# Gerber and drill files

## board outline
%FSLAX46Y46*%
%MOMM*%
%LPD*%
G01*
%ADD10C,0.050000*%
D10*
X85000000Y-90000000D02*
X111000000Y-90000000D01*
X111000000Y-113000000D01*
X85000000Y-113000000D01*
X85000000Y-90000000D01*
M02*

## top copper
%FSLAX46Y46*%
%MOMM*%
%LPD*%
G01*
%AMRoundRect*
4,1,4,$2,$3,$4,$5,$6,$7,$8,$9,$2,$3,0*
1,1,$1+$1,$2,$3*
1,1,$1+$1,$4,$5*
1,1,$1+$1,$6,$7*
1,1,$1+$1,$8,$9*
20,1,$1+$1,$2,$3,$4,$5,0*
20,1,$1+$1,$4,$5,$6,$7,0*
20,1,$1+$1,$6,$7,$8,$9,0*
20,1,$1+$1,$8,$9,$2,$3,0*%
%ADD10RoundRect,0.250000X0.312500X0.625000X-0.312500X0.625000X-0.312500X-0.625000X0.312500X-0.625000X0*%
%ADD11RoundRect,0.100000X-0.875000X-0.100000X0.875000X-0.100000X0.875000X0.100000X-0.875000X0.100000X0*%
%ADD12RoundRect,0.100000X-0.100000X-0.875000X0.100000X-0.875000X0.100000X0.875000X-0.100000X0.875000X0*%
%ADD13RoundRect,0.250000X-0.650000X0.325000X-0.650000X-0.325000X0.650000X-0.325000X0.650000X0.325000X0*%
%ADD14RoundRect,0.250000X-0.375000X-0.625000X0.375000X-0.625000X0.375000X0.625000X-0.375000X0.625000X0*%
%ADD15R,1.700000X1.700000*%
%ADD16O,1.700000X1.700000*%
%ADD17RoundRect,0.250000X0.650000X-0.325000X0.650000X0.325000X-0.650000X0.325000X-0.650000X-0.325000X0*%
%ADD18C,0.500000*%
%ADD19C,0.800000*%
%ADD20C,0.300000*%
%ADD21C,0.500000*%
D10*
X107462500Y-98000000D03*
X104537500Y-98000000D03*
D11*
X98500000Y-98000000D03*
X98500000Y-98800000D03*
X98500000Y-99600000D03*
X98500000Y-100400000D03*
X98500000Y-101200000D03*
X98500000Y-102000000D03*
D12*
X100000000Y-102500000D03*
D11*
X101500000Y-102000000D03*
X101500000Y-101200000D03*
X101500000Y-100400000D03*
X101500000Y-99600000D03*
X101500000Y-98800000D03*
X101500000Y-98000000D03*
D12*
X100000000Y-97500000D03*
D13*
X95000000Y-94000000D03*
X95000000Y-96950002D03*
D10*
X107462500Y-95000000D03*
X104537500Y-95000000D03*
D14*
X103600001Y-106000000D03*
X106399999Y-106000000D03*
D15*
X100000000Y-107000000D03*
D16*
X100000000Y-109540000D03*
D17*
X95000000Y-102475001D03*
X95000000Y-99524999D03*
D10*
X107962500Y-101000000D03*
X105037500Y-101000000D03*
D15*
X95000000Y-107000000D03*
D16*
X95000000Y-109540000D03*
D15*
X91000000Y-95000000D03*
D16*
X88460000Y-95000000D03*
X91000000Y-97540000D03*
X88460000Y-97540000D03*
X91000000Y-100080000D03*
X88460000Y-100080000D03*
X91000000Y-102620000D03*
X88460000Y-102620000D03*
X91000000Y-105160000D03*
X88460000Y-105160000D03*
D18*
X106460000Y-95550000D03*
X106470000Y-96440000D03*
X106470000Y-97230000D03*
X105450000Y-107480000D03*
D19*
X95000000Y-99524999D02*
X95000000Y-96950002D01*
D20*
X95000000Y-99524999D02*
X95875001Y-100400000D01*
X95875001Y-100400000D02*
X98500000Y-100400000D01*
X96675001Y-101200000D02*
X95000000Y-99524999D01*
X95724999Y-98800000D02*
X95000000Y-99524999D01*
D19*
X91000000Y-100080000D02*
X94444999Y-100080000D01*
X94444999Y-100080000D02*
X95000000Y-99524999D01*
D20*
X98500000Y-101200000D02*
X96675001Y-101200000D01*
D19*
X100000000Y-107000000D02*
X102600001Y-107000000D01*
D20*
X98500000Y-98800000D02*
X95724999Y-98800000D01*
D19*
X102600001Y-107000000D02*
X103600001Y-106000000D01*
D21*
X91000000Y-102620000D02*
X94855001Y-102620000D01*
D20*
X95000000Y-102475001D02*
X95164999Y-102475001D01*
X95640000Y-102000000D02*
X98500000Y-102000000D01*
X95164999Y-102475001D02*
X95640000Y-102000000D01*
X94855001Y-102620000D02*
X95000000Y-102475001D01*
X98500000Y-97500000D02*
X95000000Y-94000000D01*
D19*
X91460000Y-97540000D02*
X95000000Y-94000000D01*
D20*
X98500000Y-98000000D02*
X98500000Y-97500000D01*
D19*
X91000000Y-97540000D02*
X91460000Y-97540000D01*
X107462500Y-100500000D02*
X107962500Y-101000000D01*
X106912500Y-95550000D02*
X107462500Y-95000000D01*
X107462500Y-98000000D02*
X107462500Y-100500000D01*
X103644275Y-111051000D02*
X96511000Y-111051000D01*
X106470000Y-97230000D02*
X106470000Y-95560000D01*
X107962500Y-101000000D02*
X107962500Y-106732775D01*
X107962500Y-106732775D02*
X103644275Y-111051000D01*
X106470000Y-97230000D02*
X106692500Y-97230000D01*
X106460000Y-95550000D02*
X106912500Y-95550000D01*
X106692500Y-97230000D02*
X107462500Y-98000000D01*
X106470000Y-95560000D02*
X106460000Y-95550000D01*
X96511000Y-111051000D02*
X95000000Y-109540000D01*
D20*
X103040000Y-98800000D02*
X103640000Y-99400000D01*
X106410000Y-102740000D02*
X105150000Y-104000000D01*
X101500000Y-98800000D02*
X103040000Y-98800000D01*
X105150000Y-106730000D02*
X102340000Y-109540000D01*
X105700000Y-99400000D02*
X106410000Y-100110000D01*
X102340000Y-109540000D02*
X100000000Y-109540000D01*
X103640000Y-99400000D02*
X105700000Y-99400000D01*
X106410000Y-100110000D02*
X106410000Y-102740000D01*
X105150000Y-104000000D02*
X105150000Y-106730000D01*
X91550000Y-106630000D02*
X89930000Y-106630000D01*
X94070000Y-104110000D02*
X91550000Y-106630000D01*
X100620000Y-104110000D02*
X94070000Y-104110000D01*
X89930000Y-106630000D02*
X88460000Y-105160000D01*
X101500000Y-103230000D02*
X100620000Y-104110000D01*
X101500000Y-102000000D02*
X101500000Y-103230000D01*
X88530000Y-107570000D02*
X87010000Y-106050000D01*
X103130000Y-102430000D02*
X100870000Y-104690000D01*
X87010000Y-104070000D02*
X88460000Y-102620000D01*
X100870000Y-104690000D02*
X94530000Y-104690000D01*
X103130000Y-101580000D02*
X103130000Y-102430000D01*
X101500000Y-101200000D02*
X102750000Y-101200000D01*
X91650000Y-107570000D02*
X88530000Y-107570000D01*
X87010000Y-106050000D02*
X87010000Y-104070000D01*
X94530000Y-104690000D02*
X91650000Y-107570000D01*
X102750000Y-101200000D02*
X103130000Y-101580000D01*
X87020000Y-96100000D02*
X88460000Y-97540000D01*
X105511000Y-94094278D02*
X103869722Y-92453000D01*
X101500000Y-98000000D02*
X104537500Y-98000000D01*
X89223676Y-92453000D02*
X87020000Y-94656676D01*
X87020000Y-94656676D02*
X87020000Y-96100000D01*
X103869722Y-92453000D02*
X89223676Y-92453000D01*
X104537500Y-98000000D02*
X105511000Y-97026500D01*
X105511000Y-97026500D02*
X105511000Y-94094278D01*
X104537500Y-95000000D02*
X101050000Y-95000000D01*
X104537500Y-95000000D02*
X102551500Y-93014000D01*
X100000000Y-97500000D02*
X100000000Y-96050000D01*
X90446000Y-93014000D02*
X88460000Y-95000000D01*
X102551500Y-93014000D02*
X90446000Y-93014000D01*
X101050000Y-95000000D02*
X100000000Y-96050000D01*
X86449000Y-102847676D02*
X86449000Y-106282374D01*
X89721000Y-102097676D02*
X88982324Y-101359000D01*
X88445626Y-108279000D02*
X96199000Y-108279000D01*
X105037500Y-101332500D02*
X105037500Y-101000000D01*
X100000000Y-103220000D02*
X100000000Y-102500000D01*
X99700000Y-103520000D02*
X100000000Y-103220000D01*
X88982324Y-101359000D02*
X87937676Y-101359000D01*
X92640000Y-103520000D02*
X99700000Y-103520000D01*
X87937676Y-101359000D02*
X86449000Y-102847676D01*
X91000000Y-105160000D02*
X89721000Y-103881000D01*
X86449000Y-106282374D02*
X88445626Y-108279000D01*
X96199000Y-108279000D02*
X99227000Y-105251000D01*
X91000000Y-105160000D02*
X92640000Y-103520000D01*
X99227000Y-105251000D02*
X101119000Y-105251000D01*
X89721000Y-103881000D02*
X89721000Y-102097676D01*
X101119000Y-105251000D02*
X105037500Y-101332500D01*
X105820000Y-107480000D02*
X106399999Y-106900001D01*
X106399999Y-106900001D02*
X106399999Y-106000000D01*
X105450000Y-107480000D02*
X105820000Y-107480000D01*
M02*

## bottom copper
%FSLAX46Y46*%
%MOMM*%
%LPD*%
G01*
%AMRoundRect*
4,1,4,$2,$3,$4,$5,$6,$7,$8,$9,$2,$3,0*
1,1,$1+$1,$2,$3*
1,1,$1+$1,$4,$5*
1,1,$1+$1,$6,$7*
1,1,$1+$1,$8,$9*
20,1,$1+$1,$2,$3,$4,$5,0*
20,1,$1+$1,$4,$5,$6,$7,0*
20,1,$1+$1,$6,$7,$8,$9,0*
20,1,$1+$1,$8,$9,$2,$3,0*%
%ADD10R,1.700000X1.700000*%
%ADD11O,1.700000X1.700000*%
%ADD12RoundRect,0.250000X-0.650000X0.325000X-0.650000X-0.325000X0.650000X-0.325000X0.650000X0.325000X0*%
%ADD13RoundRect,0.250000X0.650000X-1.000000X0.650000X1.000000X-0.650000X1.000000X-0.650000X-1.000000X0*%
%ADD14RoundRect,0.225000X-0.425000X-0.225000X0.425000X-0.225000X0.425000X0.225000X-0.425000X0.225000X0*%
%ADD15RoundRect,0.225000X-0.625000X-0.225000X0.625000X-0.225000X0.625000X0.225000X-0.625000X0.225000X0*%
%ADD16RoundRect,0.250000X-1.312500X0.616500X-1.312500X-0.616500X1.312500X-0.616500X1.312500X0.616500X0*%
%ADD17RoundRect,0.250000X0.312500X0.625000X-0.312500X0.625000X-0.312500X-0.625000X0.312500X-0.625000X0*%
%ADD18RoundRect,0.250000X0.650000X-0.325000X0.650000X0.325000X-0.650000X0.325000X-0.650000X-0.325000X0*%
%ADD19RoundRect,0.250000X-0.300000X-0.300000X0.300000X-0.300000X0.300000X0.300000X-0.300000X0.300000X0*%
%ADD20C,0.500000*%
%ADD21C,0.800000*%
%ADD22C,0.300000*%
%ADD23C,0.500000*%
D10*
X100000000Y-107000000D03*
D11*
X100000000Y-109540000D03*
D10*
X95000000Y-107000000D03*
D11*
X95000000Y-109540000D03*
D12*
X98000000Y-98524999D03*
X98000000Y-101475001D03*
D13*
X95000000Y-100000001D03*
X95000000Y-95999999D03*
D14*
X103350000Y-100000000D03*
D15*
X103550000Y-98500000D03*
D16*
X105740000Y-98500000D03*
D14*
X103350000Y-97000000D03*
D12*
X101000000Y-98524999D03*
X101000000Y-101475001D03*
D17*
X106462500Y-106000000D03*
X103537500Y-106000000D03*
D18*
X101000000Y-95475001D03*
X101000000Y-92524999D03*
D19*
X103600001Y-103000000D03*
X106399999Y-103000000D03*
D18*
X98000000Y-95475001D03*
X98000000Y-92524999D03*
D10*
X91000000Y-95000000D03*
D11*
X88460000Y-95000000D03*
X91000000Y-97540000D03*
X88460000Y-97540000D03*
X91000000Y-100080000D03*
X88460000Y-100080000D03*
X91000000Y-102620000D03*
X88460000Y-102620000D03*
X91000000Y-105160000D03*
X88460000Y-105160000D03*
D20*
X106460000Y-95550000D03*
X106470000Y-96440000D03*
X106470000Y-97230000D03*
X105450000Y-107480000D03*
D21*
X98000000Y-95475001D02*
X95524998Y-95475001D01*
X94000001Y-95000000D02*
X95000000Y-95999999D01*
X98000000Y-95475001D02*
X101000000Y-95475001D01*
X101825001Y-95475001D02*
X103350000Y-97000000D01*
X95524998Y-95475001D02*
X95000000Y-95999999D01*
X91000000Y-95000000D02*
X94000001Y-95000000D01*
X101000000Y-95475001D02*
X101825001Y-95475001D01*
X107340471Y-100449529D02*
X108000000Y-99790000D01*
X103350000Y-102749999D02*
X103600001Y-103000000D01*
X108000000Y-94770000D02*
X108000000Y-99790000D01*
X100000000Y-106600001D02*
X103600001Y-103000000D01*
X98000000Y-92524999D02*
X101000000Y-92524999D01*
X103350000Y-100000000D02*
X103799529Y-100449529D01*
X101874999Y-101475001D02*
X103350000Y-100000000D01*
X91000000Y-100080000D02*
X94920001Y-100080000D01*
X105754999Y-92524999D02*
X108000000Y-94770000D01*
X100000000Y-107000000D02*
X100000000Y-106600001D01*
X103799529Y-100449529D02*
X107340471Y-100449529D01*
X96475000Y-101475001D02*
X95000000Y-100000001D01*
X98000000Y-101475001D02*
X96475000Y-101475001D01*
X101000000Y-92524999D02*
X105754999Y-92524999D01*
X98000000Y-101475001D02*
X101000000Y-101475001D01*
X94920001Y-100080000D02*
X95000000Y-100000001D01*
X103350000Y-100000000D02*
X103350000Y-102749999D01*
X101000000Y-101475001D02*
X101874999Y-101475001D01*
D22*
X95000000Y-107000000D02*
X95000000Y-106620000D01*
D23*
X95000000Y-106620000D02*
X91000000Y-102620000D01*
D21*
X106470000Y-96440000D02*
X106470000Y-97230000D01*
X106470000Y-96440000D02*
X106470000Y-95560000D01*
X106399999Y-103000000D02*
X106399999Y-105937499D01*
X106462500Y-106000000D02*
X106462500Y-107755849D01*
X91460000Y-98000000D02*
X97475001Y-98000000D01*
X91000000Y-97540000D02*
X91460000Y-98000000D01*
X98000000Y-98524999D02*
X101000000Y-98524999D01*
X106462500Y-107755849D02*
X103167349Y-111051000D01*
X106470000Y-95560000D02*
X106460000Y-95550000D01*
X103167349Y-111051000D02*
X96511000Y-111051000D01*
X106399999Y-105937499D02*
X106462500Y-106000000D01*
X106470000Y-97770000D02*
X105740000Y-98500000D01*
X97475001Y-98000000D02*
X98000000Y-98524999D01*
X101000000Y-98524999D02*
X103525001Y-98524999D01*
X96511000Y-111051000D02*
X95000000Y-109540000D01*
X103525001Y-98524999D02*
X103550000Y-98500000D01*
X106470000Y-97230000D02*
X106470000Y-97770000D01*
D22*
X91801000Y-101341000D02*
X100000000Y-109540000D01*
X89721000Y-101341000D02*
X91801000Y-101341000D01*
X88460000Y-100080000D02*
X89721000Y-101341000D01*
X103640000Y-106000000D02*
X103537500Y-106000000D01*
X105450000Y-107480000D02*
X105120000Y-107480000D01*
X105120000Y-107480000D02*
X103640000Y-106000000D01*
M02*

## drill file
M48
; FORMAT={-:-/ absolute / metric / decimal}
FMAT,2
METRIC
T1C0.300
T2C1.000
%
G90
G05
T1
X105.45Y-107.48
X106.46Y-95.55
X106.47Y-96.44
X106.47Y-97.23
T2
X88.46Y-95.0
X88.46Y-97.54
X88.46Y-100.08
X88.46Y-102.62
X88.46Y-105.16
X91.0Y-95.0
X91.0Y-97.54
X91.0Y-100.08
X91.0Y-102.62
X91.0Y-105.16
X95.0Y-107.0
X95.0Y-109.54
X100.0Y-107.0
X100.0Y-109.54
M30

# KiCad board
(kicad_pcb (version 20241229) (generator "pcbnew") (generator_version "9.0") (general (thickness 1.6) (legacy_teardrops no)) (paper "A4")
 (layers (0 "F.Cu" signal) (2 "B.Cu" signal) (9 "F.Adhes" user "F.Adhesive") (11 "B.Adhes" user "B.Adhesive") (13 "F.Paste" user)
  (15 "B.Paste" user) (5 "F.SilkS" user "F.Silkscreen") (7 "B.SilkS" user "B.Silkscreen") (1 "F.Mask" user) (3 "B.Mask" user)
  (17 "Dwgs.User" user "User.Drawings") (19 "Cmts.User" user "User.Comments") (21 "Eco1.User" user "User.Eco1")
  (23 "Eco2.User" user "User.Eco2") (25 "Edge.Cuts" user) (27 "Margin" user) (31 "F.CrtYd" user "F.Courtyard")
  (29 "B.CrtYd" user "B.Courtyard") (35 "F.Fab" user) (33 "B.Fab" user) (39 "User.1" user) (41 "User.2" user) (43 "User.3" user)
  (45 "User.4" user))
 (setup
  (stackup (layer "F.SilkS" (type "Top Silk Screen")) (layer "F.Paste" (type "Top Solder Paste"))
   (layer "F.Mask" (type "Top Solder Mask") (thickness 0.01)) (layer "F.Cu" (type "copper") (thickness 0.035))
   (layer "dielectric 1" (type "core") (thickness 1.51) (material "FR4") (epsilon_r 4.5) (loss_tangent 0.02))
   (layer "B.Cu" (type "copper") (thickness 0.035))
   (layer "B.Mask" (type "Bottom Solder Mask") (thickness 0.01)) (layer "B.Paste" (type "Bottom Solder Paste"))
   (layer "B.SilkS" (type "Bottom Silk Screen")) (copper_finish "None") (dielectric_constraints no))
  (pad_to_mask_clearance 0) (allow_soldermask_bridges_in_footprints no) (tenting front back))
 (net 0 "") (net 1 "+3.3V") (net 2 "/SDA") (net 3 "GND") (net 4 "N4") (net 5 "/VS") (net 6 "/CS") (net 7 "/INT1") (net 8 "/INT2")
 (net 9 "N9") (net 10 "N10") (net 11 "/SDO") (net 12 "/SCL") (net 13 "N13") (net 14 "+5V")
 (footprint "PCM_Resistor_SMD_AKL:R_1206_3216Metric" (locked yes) (layer "F.Cu") (at 106 98 180)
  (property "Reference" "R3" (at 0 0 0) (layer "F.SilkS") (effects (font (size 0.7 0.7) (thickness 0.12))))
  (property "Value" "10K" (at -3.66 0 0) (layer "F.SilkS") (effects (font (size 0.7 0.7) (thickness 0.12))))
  (pad "1" smd roundrect (at -1.4625 0 180) (size 1.125 1.75) (layers "F.Cu" "F.Mask" "F.Paste") (roundrect_rratio 0.222222) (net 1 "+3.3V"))
  (pad "2" smd roundrect (at 1.4625 0 180) (size 1.125 1.75) (layers "F.Cu" "F.Mask" "F.Paste") (roundrect_rratio 0.222222) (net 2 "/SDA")))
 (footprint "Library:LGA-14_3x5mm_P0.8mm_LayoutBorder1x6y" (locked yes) (layer "F.Cu") (at 100 100)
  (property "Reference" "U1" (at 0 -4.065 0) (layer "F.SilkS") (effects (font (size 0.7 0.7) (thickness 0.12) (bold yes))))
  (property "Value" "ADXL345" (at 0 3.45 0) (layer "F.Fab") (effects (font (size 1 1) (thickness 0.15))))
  (pad "1" smd roundrect (at -1.5 -2) (size 1.95 0.4) (layers "F.Cu" "F.Mask" "F.Paste") (roundrect_rratio 0.25) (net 1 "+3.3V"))
  (pad "2" smd roundrect (at -1.5 -1.2) (size 1.95 0.4) (layers "F.Cu" "F.Mask" "F.Paste") (roundrect_rratio 0.25) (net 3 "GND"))
  (pad "3" smd roundrect (at -1.5 -0.4) (size 1.95 0.4) (layers "F.Cu" "F.Mask" "F.Paste") (roundrect_rratio 0.25) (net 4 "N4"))
  (pad "4" smd roundrect (at -1.5 0.4) (size 1.95 0.4) (layers "F.Cu" "F.Mask" "F.Paste") (roundrect_rratio 0.25) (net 3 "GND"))
  (pad "5" smd roundrect (at -1.5 1.2) (size 1.95 0.4) (layers "F.Cu" "F.Mask" "F.Paste") (roundrect_rratio 0.25) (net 3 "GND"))
  (pad "6" smd roundrect (at -1.5 2) (size 1.95 0.4) (layers "F.Cu" "F.Mask" "F.Paste") (roundrect_rratio 0.25) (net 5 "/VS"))
  (pad "7" smd roundrect (at 0 2.5) (size 0.4 1.95) (layers "F.Cu" "F.Mask" "F.Paste") (roundrect_rratio 0.25) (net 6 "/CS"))
  (pad "8" smd roundrect (at 1.5 2) (size 1.95 0.4) (layers "F.Cu" "F.Mask" "F.Paste") (roundrect_rratio 0.25) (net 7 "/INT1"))
  (pad "9" smd roundrect (at 1.5 1.2) (size 1.95 0.4) (layers "F.Cu" "F.Mask" "F.Paste") (roundrect_rratio 0.25) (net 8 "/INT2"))
  (pad "10" smd roundrect (at 1.5 0.4) (size 1.95 0.4) (layers "F.Cu" "F.Mask" "F.Paste") (roundrect_rratio 0.25) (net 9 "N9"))
  (pad "11" smd roundrect (at 1.5 -0.4) (size 1.95 0.4) (layers "F.Cu" "F.Mask" "F.Paste") (roundrect_rratio 0.25) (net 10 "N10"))
  (pad "12" smd roundrect (at 1.5 -1.2) (size 1.95 0.4) (layers "F.Cu" "F.Mask" "F.Paste") (roundrect_rratio 0.25) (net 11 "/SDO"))
  (pad "13" smd roundrect (at 1.5 -2) (size 1.95 0.4) (layers "F.Cu" "F.Mask" "F.Paste") (roundrect_rratio 0.25) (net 2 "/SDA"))
  (pad "14" smd roundrect (at 0 -2.5) (size 0.4 1.95) (layers "F.Cu" "F.Mask" "F.Paste") (roundrect_rratio 0.25) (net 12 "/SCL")))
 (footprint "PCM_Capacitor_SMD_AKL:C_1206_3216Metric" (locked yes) (layer "F.Cu") (at 95 95.475001 -90)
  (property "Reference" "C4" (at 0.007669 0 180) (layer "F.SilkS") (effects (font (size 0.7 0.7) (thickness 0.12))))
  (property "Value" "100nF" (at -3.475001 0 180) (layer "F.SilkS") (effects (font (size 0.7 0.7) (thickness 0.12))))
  (pad "1" smd roundrect (at -1.475001 0 270) (size 1.15 1.8) (layers "F.Cu" "F.Mask" "F.Paste") (roundrect_rratio 0.217391) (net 1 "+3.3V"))
  (pad "2" smd roundrect (at 1.475001 0 270) (size 1.15 1.8) (layers "F.Cu" "F.Mask" "F.Paste") (roundrect_rratio 0.217391) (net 3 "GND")))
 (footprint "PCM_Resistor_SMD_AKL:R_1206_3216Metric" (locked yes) (layer "F.Cu") (at 106 95 180)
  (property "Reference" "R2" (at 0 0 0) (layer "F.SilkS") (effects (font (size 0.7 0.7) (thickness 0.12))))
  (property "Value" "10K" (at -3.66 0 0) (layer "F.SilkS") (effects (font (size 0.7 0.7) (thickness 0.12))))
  (pad "1" smd roundrect (at -1.4625 0 180) (size 1.125 1.75) (layers "F.Cu" "F.Mask" "F.Paste") (roundrect_rratio 0.222222) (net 1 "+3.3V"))
  (pad "2" smd roundrect (at 1.4625 0 180) (size 1.125 1.75) (layers "F.Cu" "F.Mask" "F.Paste") (roundrect_rratio 0.222222) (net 12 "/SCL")))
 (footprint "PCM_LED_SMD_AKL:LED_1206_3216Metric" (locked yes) (layer "F.Cu") (at 105 106)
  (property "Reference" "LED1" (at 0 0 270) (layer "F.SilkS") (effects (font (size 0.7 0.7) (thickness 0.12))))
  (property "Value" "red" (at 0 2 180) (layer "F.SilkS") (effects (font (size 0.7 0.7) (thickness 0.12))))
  (pad "1" smd roundrect (at -1.399999 0) (size 1.25 1.75) (layers "F.Cu" "F.Mask" "F.Paste") (roundrect_rratio 0.2) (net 3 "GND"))
  (pad "2" smd roundrect (at 1.399999 0) (size 1.25 1.75) (layers "F.Cu" "F.Mask" "F.Paste") (roundrect_rratio 0.2) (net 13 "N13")))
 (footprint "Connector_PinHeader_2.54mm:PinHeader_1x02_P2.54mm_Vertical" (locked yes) (layer "F.Cu") (at 100 107)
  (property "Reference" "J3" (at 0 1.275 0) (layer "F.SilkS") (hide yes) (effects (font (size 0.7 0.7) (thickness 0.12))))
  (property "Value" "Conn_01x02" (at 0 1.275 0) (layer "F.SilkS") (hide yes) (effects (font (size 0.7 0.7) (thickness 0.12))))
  (pad "1" thru_hole rect (at 0 0) (size 1.7 1.7) (drill 1) (layers "*.Cu" "*.Mask") (remove_unused_layers no) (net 3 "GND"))
  (pad "2" thru_hole oval (at 0 2.54) (size 1.7 1.7) (drill 1) (layers "*.Cu" "*.Mask") (remove_unused_layers no) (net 11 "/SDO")))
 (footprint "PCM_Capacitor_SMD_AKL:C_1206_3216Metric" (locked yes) (layer "F.Cu") (at 95 101 90)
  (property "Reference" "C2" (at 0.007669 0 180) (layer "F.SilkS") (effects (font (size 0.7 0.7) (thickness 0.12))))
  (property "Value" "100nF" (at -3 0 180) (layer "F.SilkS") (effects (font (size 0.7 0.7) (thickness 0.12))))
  (pad "1" smd roundrect (at -1.475001 0 90) (size 1.15 1.8) (layers "F.Cu" "F.Mask" "F.Paste") (roundrect_rratio 0.217391) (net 5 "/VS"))
  (pad "2" smd roundrect (at 1.475001 0 90) (size 1.15 1.8) (layers "F.Cu" "F.Mask" "F.Paste") (roundrect_rratio 0.217391) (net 3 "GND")))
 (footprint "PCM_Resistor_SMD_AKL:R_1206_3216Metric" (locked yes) (layer "F.Cu") (at 106.5 101 180)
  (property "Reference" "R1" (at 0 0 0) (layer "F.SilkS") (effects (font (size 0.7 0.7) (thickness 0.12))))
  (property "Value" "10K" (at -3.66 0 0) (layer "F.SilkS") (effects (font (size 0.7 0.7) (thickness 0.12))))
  (pad "1" smd roundrect (at -1.4625 0 180) (size 1.125 1.75) (layers "F.Cu" "F.Mask" "F.Paste") (roundrect_rratio 0.222222) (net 1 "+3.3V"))
  (pad "2" smd roundrect (at 1.4625 0 180) (size 1.125 1.75) (layers "F.Cu" "F.Mask" "F.Paste") (roundrect_rratio 0.222222) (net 6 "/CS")))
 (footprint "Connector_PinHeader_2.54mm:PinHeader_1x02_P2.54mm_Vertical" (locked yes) (layer "F.Cu") (at 95 107)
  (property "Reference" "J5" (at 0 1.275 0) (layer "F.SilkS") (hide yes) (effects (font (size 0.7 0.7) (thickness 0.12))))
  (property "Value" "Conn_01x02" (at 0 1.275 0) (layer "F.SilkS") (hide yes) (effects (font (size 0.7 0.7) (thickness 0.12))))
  (pad "1" thru_hole rect (at 0 0) (size 1.7 1.7) (drill 1) (layers "*.Cu" "*.Mask") (remove_unused_layers no) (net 5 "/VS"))
  (pad "2" thru_hole oval (at 0 2.54) (size 1.7 1.7) (drill 1) (layers "*.Cu" "*.Mask") (remove_unused_layers no) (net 1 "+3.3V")))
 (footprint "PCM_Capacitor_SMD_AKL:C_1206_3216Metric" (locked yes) (layer "B.Cu") (at 98 100 -90)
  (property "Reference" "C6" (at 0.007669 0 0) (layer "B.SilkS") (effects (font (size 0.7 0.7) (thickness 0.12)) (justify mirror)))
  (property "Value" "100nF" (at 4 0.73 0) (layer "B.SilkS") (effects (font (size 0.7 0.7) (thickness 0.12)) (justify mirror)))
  (pad "1" smd roundrect (at -1.475001 0 270) (size 1.15 1.8) (layers "B.Cu" "B.Mask" "B.Paste") (roundrect_rratio 0.217391) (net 1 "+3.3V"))
  (pad "2" smd roundrect (at 1.475001 0 270) (size 1.15 1.8) (layers "B.Cu" "B.Mask" "B.Paste") (roundrect_rratio 0.217391) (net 3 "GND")))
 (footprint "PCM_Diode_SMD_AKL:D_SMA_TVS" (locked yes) (layer "B.Cu") (at 95 98 90)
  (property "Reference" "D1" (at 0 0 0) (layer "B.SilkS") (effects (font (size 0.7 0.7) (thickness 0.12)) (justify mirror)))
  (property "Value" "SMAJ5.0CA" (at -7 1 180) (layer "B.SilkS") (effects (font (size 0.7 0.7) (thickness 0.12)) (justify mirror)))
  (pad "1" smd roundrect (at -2.000001 0 90) (size 2.5 1.8) (layers "B.Cu" "B.Mask" "B.Paste") (roundrect_rratio 0.1388888889) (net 3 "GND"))
  (pad "2" smd roundrect (at 2.000001 0 90) (size 2.5 1.8) (layers "B.Cu" "B.Mask" "B.Paste") (roundrect_rratio 0.1388888889) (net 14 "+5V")))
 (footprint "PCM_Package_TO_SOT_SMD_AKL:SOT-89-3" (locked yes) (layer "B.Cu") (at 105 98.5)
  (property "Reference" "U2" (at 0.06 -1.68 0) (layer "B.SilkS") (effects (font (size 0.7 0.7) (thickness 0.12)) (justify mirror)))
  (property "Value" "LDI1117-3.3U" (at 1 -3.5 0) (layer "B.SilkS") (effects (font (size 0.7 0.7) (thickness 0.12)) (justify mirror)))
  (pad "1" smd roundrect (at -1.65 1.5) (size 1.3 0.9) (layers "B.Cu" "B.Mask" "B.Paste") (roundrect_rratio 0.25) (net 3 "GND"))
  (pad "2" smd roundrect (at -1.45 0) (size 1.7 0.9) (layers "B.Cu" "B.Mask" "B.Paste") (roundrect_rratio 0.25) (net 1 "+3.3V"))
  (pad "2" smd roundrect (at 0.74 0 270) (size 1.733 3.125) (layers "B.Cu" "B.Mask" "B.Paste") (roundrect_rratio 0.1442585113)
   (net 1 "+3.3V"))
  (pad "3" smd roundrect (at -1.65 -1.5) (size 1.3 0.9) (layers "B.Cu" "B.Mask" "B.Paste") (roundrect_rratio 0.25) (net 14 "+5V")))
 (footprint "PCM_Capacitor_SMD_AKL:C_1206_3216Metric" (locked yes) (layer "B.Cu") (at 101 100 -90)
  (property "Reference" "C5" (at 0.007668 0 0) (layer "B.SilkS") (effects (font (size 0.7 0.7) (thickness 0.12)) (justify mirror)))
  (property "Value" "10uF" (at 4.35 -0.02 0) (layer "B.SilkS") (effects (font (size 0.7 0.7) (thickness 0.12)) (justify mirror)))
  (pad "1" smd roundrect (at -1.475001 0 270) (size 1.15 1.8) (layers "B.Cu" "B.Mask" "B.Paste") (roundrect_rratio 0.217391) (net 1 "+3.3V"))
  (pad "2" smd roundrect (at 1.475001 0 270) (size 1.15 1.8) (layers "B.Cu" "B.Mask" "B.Paste") (roundrect_rratio 0.217391) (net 3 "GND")))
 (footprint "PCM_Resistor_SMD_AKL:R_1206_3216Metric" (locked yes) (layer "B.Cu") (at 105 106 180)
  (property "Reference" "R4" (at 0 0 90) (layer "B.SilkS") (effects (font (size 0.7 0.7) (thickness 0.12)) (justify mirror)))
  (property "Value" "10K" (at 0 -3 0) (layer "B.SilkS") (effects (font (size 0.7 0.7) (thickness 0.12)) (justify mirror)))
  (pad "1" smd roundrect (at -1.4625 0 180) (size 1.125 1.75) (layers "B.Cu" "B.Mask" "B.Paste") (roundrect_rratio 0.222222) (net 1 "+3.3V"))
  (pad "2" smd roundrect (at 1.4625 0 180) (size 1.125 1.75) (layers "B.Cu" "B.Mask" "B.Paste") (roundrect_rratio 0.222222) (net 13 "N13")))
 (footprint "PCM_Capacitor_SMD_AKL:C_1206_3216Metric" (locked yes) (layer "B.Cu") (at 101 94 90)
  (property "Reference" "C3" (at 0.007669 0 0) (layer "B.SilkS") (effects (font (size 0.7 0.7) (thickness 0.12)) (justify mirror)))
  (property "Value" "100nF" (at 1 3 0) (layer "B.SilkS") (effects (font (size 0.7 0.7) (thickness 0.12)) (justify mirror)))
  (pad "1" smd roundrect (at -1.475001 0 90) (size 1.15 1.8) (layers "B.Cu" "B.Mask" "B.Paste") (roundrect_rratio 0.217391) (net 14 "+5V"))
  (pad "2" smd roundrect (at 1.475001 0 90) (size 1.15 1.8) (layers "B.Cu" "B.Mask" "B.Paste") (roundrect_rratio 0.217391) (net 3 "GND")))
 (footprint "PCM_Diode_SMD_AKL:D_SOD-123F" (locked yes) (layer "B.Cu") (at 105 103)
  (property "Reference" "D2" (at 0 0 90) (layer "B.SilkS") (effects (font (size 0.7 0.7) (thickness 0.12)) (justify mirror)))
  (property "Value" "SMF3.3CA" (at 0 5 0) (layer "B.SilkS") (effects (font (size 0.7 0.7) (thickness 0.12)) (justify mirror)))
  (pad "1" smd roundrect (at -1.399999 0) (size 1.1 1.1) (layers "B.Cu" "B.Mask" "B.Paste") (roundrect_rratio 0.2272727273) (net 3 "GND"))
  (pad "2" smd roundrect (at 1.399999 0) (size 1.1 1.1) (layers "B.Cu" "B.Mask" "B.Paste") (roundrect_rratio 0.2272727273) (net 1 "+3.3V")))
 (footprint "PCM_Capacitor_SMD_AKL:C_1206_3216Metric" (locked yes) (layer "B.Cu") (at 98 94 90)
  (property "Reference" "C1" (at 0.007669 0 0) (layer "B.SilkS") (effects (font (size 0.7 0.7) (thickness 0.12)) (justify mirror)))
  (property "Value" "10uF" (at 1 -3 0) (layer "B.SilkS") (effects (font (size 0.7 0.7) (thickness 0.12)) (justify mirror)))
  (pad "1" smd roundrect (at -1.475001 0 90) (size 1.15 1.8) (layers "B.Cu" "B.Mask" "B.Paste") (roundrect_rratio 0.217391) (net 14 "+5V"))
  (pad "2" smd roundrect (at 1.475001 0 90) (size 1.15 1.8) (layers "B.Cu" "B.Mask" "B.Paste") (roundrect_rratio 0.217391) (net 3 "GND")))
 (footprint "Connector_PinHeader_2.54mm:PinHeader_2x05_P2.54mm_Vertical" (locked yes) (layer "B.Cu") (at 91 95 180)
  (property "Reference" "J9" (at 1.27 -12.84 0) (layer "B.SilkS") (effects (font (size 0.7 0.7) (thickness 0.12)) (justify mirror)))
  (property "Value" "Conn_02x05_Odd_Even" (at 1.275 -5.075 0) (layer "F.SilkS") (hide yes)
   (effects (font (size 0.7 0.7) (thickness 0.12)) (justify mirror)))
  (pad "1" thru_hole rect (at 0 0 180) (size 1.7 1.7) (drill 1) (layers "*.Cu" "*.Mask") (remove_unused_layers no) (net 14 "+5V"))
  (pad "2" thru_hole oval (at 2.54 0 180) (size 1.7 1.7) (drill 1) (layers "*.Cu" "*.Mask") (remove_unused_layers no) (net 12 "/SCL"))
  (pad "3" thru_hole oval (at 0 -2.54 180) (size 1.7 1.7) (drill 1) (layers "*.Cu" "*.Mask") (remove_unused_layers no) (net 1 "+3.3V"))
  (pad "4" thru_hole oval (at 2.54 -2.54 180) (size 1.7 1.7) (drill 1) (layers "*.Cu" "*.Mask") (remove_unused_layers no) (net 2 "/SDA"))
  (pad "5" thru_hole oval (at 0 -5.08 180) (size 1.7 1.7) (drill 1) (layers "*.Cu" "*.Mask") (remove_unused_layers no) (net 3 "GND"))
  (pad "6" thru_hole oval (at 2.54 -5.08 180) (size 1.7 1.7) (drill 1) (layers "*.Cu" "*.Mask") (remove_unused_layers no) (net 11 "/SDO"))
  (pad "7" thru_hole oval (at 0 -7.62 180) (size 1.7 1.7) (drill 1) (layers "*.Cu" "*.Mask") (remove_unused_layers no) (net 5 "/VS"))
  (pad "8" thru_hole oval (at 2.54 -7.62 180) (size 1.7 1.7) (drill 1) (layers "*.Cu" "*.Mask") (remove_unused_layers no) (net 8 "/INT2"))
  (pad "9" thru_hole oval (at 0 -10.16 180) (size 1.7 1.7) (drill 1) (layers "*.Cu" "*.Mask") (remove_unused_layers no) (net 6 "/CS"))
  (pad "10" thru_hole oval (at 2.54 -10.16 180) (size 1.7 1.7) (drill 1) (layers "*.Cu" "*.Mask") (remove_unused_layers no) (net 7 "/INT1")))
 (gr_rect (start 85 90) (end 111 113) (stroke (width 0.05) (type default)) (fill no) (locked yes) (layer "Edge.Cuts"))
 (segment (start 98 95.475001) (end 95.524998 95.475001) (width 0.8) (locked yes) (layer "B.Cu") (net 14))
 (segment (start 94.000001 95) (end 95 95.999999) (width 0.8) (locked yes) (layer "B.Cu") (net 14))
 (segment (start 98 95.475001) (end 101 95.475001) (width 0.8) (locked yes) (layer "B.Cu") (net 14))
 (segment (start 101.825001 95.475001) (end 103.35 97) (width 0.8) (locked yes) (layer "B.Cu") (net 14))
 (segment (start 95.524998 95.475001) (end 95 95.999999) (width 0.8) (locked yes) (layer "B.Cu") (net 14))
 (segment (start 91 95) (end 94.000001 95) (width 0.8) (locked yes) (layer "B.Cu") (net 14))
 (segment (start 101 95.475001) (end 101.825001 95.475001) (width 0.8) (locked yes) (layer "B.Cu") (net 14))
 (segment (start 95 99.524999) (end 95 96.950002) (width 0.8) (locked yes) (layer "F.Cu") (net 3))
 (segment (start 95 99.524999) (end 95.875001 100.4) (width 0.3) (locked yes) (layer "F.Cu") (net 3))
 (segment (start 95.875001 100.4) (end 98.5 100.4) (width 0.3) (locked yes) (layer "F.Cu") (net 3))
 (segment (start 96.675001 101.2) (end 95 99.524999) (width 0.3) (locked yes) (layer "F.Cu") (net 3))
 (segment (start 95.724999 98.8) (end 95 99.524999) (width 0.3) (locked yes) (layer "F.Cu") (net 3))
 (segment (start 91 100.08) (end 94.444999 100.08) (width 0.8) (locked yes) (layer "F.Cu") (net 3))
 (segment (start 94.444999 100.08) (end 95 99.524999) (width 0.8) (locked yes) (layer "F.Cu") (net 3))
 (segment (start 98.5 101.2) (end 96.675001 101.2) (width 0.3) (locked yes) (layer "F.Cu") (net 3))
 (segment (start 100 107) (end 102.600001 107) (width 0.8) (locked yes) (layer "F.Cu") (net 3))
 (segment (start 98.5 98.8) (end 95.724999 98.8) (width 0.3) (locked yes) (layer "F.Cu") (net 3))
 (segment (start 102.600001 107) (end 103.600001 106) (width 0.8) (locked yes) (layer "F.Cu") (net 3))
 (segment (start 107.340471 100.449529) (end 108 99.79) (width 0.8) (locked yes) (layer "B.Cu") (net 3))
 (segment (start 103.35 102.749999) (end 103.600001 103) (width 0.8) (locked yes) (layer "B.Cu") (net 3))
 (segment (start 108 94.77) (end 108 99.79) (width 0.8) (locked yes) (layer "B.Cu") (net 3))
 (segment (start 100 106.600001) (end 103.600001 103) (width 0.8) (locked yes) (layer "B.Cu") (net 3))
 (segment (start 98 92.524999) (end 101 92.524999) (width 0.8) (locked yes) (layer "B.Cu") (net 3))
 (segment (start 103.35 100) (end 103.799529 100.449529) (width 0.8) (locked yes) (layer "B.Cu") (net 3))
 (segment (start 101.874999 101.475001) (end 103.35 100) (width 0.8) (locked yes) (layer "B.Cu") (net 3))
 (segment (start 91 100.08) (end 94.920001 100.08) (width 0.8) (locked yes) (layer "B.Cu") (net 3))
 (segment (start 105.754999 92.524999) (end 108 94.77) (width 0.8) (locked yes) (layer "B.Cu") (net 3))
 (segment (start 100 107) (end 100 106.600001) (width 0.8) (locked yes) (layer "B.Cu") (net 3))
 (segment (start 103.799529 100.449529) (end 107.340471 100.449529) (width 0.8) (locked yes) (layer "B.Cu") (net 3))
 (segment (start 96.475 101.475001) (end 95 100.000001) (width 0.8) (locked yes) (layer "B.Cu") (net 3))
 (segment (start 98 101.475001) (end 96.475 101.475001) (width 0.8) (locked yes) (layer "B.Cu") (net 3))
 (segment (start 101 92.524999) (end 105.754999 92.524999) (width 0.8) (locked yes) (layer "B.Cu") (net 3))
 (segment (start 98 101.475001) (end 101 101.475001) (width 0.8) (locked yes) (layer "B.Cu") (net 3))
 (segment (start 94.920001 100.08) (end 95 100.000001) (width 0.8) (locked yes) (layer "B.Cu") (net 3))
 (segment (start 103.35 100) (end 103.35 102.749999) (width 0.8) (locked yes) (layer "B.Cu") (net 3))
 (segment (start 101 101.475001) (end 101.874999 101.475001) (width 0.8) (locked yes) (layer "B.Cu") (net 3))
 (segment (start 91 102.62) (end 94.855001 102.62) (width 0.5) (locked yes) (layer "F.Cu") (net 5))
 (segment (start 95 102.475001) (end 95.164999 102.475001) (width 0.3) (locked yes) (layer "F.Cu") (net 5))
 (segment (start 95.64 102) (end 98.5 102) (width 0.3) (locked yes) (layer "F.Cu") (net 5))
 (segment (start 95.164999 102.475001) (end 95.64 102) (width 0.3) (locked yes) (layer "F.Cu") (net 5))
 (segment (start 94.855001 102.62) (end 95 102.475001) (width 0.3) (locked yes) (layer "F.Cu") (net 5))
 (segment (start 95 107) (end 95 106.62) (width 0.3) (locked yes) (layer "B.Cu") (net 5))
 (segment (start 95 106.62) (end 91 102.62) (width 0.5) (locked yes) (layer "B.Cu") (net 5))
 (segment (start 98.5 97.5) (end 95 94) (width 0.3) (locked yes) (layer "F.Cu") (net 1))
 (segment (start 91.46 97.54) (end 95 94) (width 0.8) (locked yes) (layer "F.Cu") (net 1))
 (segment (start 98.5 98) (end 98.5 97.5) (width 0.3) (locked yes) (layer "F.Cu") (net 1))
 (segment (start 91 97.54) (end 91.46 97.54) (width 0.8) (locked yes) (layer "F.Cu") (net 1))
 (segment (start 107.4625 100.5) (end 107.9625 101) (width 0.8) (locked yes) (layer "F.Cu") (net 1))
 (segment (start 106.9125 95.55) (end 107.4625 95) (width 0.8) (locked yes) (layer "F.Cu") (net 1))
 (segment (start 107.4625 98) (end 107.4625 100.5) (width 0.8) (locked yes) (layer "F.Cu") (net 1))
 (segment (start 103.644275 111.051) (end 96.511 111.051) (width 0.8) (locked yes) (layer "F.Cu") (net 1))
 (segment (start 106.47 97.23) (end 106.47 95.56) (width 0.8) (locked yes) (layer "F.Cu") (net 1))
 (segment (start 107.9625 101) (end 107.9625 106.732775) (width 0.8) (locked yes) (layer "F.Cu") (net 1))
 (segment (start 107.9625 106.732775) (end 103.644275 111.051) (width 0.8) (locked yes) (layer "F.Cu") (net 1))
 (segment (start 106.47 97.23) (end 106.6925 97.23) (width 0.8) (locked yes) (layer "F.Cu") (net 1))
 (segment (start 106.46 95.55) (end 106.9125 95.55) (width 0.8) (locked yes) (layer "F.Cu") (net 1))
 (segment (start 106.6925 97.23) (end 107.4625 98) (width 0.8) (locked yes) (layer "F.Cu") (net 1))
 (segment (start 106.47 95.56) (end 106.46 95.55) (width 0.8) (locked yes) (layer "F.Cu") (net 1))
 (segment (start 96.511 111.051) (end 95 109.54) (width 0.8) (locked yes) (layer "F.Cu") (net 1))
 (via (at 106.46 95.55) (size 0.5) (drill 0.3) (layers "F.Cu" "B.Cu") (locked yes) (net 1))
 (via (at 106.47 96.44) (size 0.5) (drill 0.3) (layers "F.Cu" "B.Cu") (locked yes) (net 1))
 (via (at 106.47 97.23) (size 0.5) (drill 0.3) (layers "F.Cu" "B.Cu") (locked yes) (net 1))
 (segment (start 106.47 96.44) (end 106.47 97.23) (width 0.8) (locked yes) (layer "B.Cu") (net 1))
 (segment (start 106.47 96.44) (end 106.47 95.56) (width 0.8) (locked yes) (layer "B.Cu") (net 1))
 (segment (start 106.399999 103) (end 106.399999 105.937499) (width 0.8) (locked yes) (layer "B.Cu") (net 1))
 (segment (start 106.4625 106) (end 106.4625 107.755849) (width 0.8) (locked yes) (layer "B.Cu") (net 1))
 (segment (start 91.46 98) (end 97.475001 98) (width 0.8) (locked yes) (layer "B.Cu") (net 1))
 (segment (start 91 97.54) (end 91.46 98) (width 0.8) (locked yes) (layer "B.Cu") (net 1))
 (segment (start 98 98.524999) (end 101 98.524999) (width 0.8) (locked yes) (layer "B.Cu") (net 1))
 (segment (start 106.4625 107.755849) (end 103.167349 111.051) (width 0.8) (locked yes) (layer "B.Cu") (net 1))
 (segment (start 106.47 95.56) (end 106.46 95.55) (width 0.8) (locked yes) (layer "B.Cu") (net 1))
 (segment (start 103.167349 111.051) (end 96.511 111.051) (width 0.8) (locked yes) (layer "B.Cu") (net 1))
 (segment (start 106.399999 105.937499) (end 106.4625 106) (width 0.8) (locked yes) (layer "B.Cu") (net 1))
 (segment (start 106.47 97.77) (end 105.74 98.5) (width 0.8) (locked yes) (layer "B.Cu") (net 1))
 (segment (start 97.475001 98) (end 98 98.524999) (width 0.8) (locked yes) (layer "B.Cu") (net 1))
 (segment (start 101 98.524999) (end 103.525001 98.524999) (width 0.8) (locked yes) (layer "B.Cu") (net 1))
 (segment (start 96.511 111.051) (end 95 109.54) (width 0.8) (locked yes) (layer "B.Cu") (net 1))
 (segment (start 103.525001 98.524999) (end 103.55 98.5) (width 0.8) (locked yes) (layer "B.Cu") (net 1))
 (segment (start 106.47 97.23) (end 106.47 97.77) (width 0.8) (locked yes) (layer "B.Cu") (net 1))
 (segment (start 103.04 98.8) (end 103.64 99.4) (width 0.3) (locked yes) (layer "F.Cu") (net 11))
 (segment (start 106.41 102.74) (end 105.15 104) (width 0.3) (locked yes) (layer "F.Cu") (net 11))
 (segment (start 101.5 98.8) (end 103.04 98.8) (width 0.3) (locked yes) (layer "F.Cu") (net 11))
 (segment (start 105.15 106.73) (end 102.34 109.54) (width 0.3) (locked yes) (layer "F.Cu") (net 11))
 (segment (start 105.7 99.4) (end 106.41 100.11) (width 0.3) (locked yes) (layer "F.Cu") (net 11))
 (segment (start 102.34 109.54) (end 100 109.54) (width 0.3) (locked yes) (layer "F.Cu") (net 11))
 (segment (start 103.64 99.4) (end 105.7 99.4) (width 0.3) (locked yes) (layer "F.Cu") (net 11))
 (segment (start 106.41 100.11) (end 106.41 102.74) (width 0.3) (locked yes) (layer "F.Cu") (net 11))
 (segment (start 105.15 104) (end 105.15 106.73) (width 0.3) (locked yes) (layer "F.Cu") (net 11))
 (segment (start 91.801 101.341) (end 100 109.54) (width 0.3) (locked yes) (layer "B.Cu") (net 11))
 (segment (start 89.721 101.341) (end 91.801 101.341) (width 0.3) (locked yes) (layer "B.Cu") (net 11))
 (segment (start 88.46 100.08) (end 89.721 101.341) (width 0.3) (locked yes) (layer "B.Cu") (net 11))
 (segment (start 91.55 106.63) (end 89.93 106.63) (width 0.3) (locked yes) (layer "F.Cu") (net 7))
 (segment (start 94.07 104.11) (end 91.55 106.63) (width 0.3) (locked yes) (layer "F.Cu") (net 7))
 (segment (start 100.62 104.11) (end 94.07 104.11) (width 0.3) (locked yes) (layer "F.Cu") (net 7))
 (segment (start 89.93 106.63) (end 88.46 105.16) (width 0.3) (locked yes) (layer "F.Cu") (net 7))
 (segment (start 101.5 103.23) (end 100.62 104.11) (width 0.3) (locked yes) (layer "F.Cu") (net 7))
 (segment (start 101.5 102) (end 101.5 103.23) (width 0.3) (locked yes) (layer "F.Cu") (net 7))
 (segment (start 88.53 107.57) (end 87.01 106.05) (width 0.3) (locked yes) (layer "F.Cu") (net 8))
 (segment (start 103.13 102.43) (end 100.87 104.69) (width 0.3) (locked yes) (layer "F.Cu") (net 8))
 (segment (start 87.01 104.07) (end 88.46 102.62) (width 0.3) (locked yes) (layer "F.Cu") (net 8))
 (segment (start 100.87 104.69) (end 94.53 104.69) (width 0.3) (locked yes) (layer "F.Cu") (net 8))
 (segment (start 103.13 101.58) (end 103.13 102.43) (width 0.3) (locked yes) (layer "F.Cu") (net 8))
 (segment (start 101.5 101.2) (end 102.75 101.2) (width 0.3) (locked yes) (layer "F.Cu") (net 8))
 (segment (start 91.65 107.57) (end 88.53 107.57) (width 0.3) (locked yes) (layer "F.Cu") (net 8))
 (segment (start 87.01 106.05) (end 87.01 104.07) (width 0.3) (locked yes) (layer "F.Cu") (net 8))
 (segment (start 94.53 104.69) (end 91.65 107.57) (width 0.3) (locked yes) (layer "F.Cu") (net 8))
 (segment (start 102.75 101.2) (end 103.13 101.58) (width 0.3) (locked yes) (layer "F.Cu") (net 8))
 (segment (start 87.02 96.1) (end 88.46 97.54) (width 0.3) (locked yes) (layer "F.Cu") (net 2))
 (segment (start 105.511 94.094278) (end 103.869722 92.453) (width 0.3) (locked yes) (layer "F.Cu") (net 2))
 (segment (start 101.5 98) (end 104.5375 98) (width 0.3) (locked yes) (layer "F.Cu") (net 2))
 (segment (start 89.223676 92.453) (end 87.02 94.656676) (width 0.3) (locked yes) (layer "F.Cu") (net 2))
 (segment (start 87.02 94.656676) (end 87.02 96.1) (width 0.3) (locked yes) (layer "F.Cu") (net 2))
 (segment (start 103.869722 92.453) (end 89.223676 92.453) (width 0.3) (locked yes) (layer "F.Cu") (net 2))
 (segment (start 104.5375 98) (end 105.511 97.0265) (width 0.3) (locked yes) (layer "F.Cu") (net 2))
 (segment (start 105.511 97.0265) (end 105.511 94.094278) (width 0.3) (locked yes) (layer "F.Cu") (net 2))
 (segment (start 104.5375 95) (end 101.05 95) (width 0.3) (locked yes) (layer "F.Cu") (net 12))
 (segment (start 104.5375 95) (end 102.5515 93.014) (width 0.3) (locked yes) (layer "F.Cu") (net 12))
 (segment (start 100 97.5) (end 100 96.05) (width 0.3) (locked yes) (layer "F.Cu") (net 12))
 (segment (start 90.446 93.014) (end 88.46 95) (width 0.3) (locked yes) (layer "F.Cu") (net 12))
 (segment (start 102.5515 93.014) (end 90.446 93.014) (width 0.3) (locked yes) (layer "F.Cu") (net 12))
 (segment (start 101.05 95) (end 100 96.05) (width 0.3) (locked yes) (layer "F.Cu") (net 12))
 (segment (start 86.449 102.847676) (end 86.449 106.282374) (width 0.3) (locked yes) (layer "F.Cu") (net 6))
 (segment (start 89.721 102.097676) (end 88.982324 101.359) (width 0.3) (locked yes) (layer "F.Cu") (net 6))
 (segment (start 88.445626 108.279) (end 96.199 108.279) (width 0.3) (locked yes) (layer "F.Cu") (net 6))
 (segment (start 105.0375 101.3325) (end 105.0375 101) (width 0.3) (locked yes) (layer "F.Cu") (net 6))
 (segment (start 100 103.22) (end 100 102.5) (width 0.3) (locked yes) (layer "F.Cu") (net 6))
 (segment (start 99.7 103.52) (end 100 103.22) (width 0.3) (locked yes) (layer "F.Cu") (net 6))
 (segment (start 88.982324 101.359) (end 87.937676 101.359) (width 0.3) (locked yes) (layer "F.Cu") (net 6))
 (segment (start 92.64 103.52) (end 99.7 103.52) (width 0.3) (locked yes) (layer "F.Cu") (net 6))
 (segment (start 87.937676 101.359) (end 86.449 102.847676) (width 0.3) (locked yes) (layer "F.Cu") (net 6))
 (segment (start 91 105.16) (end 89.721 103.881) (width 0.3) (locked yes) (layer "F.Cu") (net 6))
 (segment (start 86.449 106.282374) (end 88.445626 108.279) (width 0.3) (locked yes) (layer "F.Cu") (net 6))
 (segment (start 96.199 108.279) (end 99.227 105.251) (width 0.3) (locked yes) (layer "F.Cu") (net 6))
 (segment (start 91 105.16) (end 92.64 103.52) (width 0.3) (locked yes) (layer "F.Cu") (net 6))
 (segment (start 99.227 105.251) (end 101.119 105.251) (width 0.3) (locked yes) (layer "F.Cu") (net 6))
 (segment (start 89.721 103.881) (end 89.721 102.097676) (width 0.3) (locked yes) (layer "F.Cu") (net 6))
 (segment (start 101.119 105.251) (end 105.0375 101.3325) (width 0.3) (locked yes) (layer "F.Cu") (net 6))
 (segment (start 105.82 107.48) (end 106.399999 106.900001) (width 0.3) (locked yes) (layer "F.Cu") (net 13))
 (segment (start 106.399999 106.900001) (end 106.399999 106) (width 0.3) (locked yes) (layer "F.Cu") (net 13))
 (segment (start 105.45 107.48) (end 105.82 107.48) (width 0.3) (locked yes) (layer "F.Cu") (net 13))
 (via (at 105.45 107.48) (size 0.5) (drill 0.3) (layers "F.Cu" "B.Cu") (locked yes) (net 13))
 (segment (start 103.64 106) (end 103.5375 106) (width 0.3) (locked yes) (layer "B.Cu") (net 13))
 (segment (start 105.45 107.48) (end 105.12 107.48) (width 0.3) (locked yes) (layer "B.Cu") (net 13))
 (segment (start 105.12 107.48) (end 103.64 106) (width 0.3) (locked yes) (layer "B.Cu") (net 13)))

